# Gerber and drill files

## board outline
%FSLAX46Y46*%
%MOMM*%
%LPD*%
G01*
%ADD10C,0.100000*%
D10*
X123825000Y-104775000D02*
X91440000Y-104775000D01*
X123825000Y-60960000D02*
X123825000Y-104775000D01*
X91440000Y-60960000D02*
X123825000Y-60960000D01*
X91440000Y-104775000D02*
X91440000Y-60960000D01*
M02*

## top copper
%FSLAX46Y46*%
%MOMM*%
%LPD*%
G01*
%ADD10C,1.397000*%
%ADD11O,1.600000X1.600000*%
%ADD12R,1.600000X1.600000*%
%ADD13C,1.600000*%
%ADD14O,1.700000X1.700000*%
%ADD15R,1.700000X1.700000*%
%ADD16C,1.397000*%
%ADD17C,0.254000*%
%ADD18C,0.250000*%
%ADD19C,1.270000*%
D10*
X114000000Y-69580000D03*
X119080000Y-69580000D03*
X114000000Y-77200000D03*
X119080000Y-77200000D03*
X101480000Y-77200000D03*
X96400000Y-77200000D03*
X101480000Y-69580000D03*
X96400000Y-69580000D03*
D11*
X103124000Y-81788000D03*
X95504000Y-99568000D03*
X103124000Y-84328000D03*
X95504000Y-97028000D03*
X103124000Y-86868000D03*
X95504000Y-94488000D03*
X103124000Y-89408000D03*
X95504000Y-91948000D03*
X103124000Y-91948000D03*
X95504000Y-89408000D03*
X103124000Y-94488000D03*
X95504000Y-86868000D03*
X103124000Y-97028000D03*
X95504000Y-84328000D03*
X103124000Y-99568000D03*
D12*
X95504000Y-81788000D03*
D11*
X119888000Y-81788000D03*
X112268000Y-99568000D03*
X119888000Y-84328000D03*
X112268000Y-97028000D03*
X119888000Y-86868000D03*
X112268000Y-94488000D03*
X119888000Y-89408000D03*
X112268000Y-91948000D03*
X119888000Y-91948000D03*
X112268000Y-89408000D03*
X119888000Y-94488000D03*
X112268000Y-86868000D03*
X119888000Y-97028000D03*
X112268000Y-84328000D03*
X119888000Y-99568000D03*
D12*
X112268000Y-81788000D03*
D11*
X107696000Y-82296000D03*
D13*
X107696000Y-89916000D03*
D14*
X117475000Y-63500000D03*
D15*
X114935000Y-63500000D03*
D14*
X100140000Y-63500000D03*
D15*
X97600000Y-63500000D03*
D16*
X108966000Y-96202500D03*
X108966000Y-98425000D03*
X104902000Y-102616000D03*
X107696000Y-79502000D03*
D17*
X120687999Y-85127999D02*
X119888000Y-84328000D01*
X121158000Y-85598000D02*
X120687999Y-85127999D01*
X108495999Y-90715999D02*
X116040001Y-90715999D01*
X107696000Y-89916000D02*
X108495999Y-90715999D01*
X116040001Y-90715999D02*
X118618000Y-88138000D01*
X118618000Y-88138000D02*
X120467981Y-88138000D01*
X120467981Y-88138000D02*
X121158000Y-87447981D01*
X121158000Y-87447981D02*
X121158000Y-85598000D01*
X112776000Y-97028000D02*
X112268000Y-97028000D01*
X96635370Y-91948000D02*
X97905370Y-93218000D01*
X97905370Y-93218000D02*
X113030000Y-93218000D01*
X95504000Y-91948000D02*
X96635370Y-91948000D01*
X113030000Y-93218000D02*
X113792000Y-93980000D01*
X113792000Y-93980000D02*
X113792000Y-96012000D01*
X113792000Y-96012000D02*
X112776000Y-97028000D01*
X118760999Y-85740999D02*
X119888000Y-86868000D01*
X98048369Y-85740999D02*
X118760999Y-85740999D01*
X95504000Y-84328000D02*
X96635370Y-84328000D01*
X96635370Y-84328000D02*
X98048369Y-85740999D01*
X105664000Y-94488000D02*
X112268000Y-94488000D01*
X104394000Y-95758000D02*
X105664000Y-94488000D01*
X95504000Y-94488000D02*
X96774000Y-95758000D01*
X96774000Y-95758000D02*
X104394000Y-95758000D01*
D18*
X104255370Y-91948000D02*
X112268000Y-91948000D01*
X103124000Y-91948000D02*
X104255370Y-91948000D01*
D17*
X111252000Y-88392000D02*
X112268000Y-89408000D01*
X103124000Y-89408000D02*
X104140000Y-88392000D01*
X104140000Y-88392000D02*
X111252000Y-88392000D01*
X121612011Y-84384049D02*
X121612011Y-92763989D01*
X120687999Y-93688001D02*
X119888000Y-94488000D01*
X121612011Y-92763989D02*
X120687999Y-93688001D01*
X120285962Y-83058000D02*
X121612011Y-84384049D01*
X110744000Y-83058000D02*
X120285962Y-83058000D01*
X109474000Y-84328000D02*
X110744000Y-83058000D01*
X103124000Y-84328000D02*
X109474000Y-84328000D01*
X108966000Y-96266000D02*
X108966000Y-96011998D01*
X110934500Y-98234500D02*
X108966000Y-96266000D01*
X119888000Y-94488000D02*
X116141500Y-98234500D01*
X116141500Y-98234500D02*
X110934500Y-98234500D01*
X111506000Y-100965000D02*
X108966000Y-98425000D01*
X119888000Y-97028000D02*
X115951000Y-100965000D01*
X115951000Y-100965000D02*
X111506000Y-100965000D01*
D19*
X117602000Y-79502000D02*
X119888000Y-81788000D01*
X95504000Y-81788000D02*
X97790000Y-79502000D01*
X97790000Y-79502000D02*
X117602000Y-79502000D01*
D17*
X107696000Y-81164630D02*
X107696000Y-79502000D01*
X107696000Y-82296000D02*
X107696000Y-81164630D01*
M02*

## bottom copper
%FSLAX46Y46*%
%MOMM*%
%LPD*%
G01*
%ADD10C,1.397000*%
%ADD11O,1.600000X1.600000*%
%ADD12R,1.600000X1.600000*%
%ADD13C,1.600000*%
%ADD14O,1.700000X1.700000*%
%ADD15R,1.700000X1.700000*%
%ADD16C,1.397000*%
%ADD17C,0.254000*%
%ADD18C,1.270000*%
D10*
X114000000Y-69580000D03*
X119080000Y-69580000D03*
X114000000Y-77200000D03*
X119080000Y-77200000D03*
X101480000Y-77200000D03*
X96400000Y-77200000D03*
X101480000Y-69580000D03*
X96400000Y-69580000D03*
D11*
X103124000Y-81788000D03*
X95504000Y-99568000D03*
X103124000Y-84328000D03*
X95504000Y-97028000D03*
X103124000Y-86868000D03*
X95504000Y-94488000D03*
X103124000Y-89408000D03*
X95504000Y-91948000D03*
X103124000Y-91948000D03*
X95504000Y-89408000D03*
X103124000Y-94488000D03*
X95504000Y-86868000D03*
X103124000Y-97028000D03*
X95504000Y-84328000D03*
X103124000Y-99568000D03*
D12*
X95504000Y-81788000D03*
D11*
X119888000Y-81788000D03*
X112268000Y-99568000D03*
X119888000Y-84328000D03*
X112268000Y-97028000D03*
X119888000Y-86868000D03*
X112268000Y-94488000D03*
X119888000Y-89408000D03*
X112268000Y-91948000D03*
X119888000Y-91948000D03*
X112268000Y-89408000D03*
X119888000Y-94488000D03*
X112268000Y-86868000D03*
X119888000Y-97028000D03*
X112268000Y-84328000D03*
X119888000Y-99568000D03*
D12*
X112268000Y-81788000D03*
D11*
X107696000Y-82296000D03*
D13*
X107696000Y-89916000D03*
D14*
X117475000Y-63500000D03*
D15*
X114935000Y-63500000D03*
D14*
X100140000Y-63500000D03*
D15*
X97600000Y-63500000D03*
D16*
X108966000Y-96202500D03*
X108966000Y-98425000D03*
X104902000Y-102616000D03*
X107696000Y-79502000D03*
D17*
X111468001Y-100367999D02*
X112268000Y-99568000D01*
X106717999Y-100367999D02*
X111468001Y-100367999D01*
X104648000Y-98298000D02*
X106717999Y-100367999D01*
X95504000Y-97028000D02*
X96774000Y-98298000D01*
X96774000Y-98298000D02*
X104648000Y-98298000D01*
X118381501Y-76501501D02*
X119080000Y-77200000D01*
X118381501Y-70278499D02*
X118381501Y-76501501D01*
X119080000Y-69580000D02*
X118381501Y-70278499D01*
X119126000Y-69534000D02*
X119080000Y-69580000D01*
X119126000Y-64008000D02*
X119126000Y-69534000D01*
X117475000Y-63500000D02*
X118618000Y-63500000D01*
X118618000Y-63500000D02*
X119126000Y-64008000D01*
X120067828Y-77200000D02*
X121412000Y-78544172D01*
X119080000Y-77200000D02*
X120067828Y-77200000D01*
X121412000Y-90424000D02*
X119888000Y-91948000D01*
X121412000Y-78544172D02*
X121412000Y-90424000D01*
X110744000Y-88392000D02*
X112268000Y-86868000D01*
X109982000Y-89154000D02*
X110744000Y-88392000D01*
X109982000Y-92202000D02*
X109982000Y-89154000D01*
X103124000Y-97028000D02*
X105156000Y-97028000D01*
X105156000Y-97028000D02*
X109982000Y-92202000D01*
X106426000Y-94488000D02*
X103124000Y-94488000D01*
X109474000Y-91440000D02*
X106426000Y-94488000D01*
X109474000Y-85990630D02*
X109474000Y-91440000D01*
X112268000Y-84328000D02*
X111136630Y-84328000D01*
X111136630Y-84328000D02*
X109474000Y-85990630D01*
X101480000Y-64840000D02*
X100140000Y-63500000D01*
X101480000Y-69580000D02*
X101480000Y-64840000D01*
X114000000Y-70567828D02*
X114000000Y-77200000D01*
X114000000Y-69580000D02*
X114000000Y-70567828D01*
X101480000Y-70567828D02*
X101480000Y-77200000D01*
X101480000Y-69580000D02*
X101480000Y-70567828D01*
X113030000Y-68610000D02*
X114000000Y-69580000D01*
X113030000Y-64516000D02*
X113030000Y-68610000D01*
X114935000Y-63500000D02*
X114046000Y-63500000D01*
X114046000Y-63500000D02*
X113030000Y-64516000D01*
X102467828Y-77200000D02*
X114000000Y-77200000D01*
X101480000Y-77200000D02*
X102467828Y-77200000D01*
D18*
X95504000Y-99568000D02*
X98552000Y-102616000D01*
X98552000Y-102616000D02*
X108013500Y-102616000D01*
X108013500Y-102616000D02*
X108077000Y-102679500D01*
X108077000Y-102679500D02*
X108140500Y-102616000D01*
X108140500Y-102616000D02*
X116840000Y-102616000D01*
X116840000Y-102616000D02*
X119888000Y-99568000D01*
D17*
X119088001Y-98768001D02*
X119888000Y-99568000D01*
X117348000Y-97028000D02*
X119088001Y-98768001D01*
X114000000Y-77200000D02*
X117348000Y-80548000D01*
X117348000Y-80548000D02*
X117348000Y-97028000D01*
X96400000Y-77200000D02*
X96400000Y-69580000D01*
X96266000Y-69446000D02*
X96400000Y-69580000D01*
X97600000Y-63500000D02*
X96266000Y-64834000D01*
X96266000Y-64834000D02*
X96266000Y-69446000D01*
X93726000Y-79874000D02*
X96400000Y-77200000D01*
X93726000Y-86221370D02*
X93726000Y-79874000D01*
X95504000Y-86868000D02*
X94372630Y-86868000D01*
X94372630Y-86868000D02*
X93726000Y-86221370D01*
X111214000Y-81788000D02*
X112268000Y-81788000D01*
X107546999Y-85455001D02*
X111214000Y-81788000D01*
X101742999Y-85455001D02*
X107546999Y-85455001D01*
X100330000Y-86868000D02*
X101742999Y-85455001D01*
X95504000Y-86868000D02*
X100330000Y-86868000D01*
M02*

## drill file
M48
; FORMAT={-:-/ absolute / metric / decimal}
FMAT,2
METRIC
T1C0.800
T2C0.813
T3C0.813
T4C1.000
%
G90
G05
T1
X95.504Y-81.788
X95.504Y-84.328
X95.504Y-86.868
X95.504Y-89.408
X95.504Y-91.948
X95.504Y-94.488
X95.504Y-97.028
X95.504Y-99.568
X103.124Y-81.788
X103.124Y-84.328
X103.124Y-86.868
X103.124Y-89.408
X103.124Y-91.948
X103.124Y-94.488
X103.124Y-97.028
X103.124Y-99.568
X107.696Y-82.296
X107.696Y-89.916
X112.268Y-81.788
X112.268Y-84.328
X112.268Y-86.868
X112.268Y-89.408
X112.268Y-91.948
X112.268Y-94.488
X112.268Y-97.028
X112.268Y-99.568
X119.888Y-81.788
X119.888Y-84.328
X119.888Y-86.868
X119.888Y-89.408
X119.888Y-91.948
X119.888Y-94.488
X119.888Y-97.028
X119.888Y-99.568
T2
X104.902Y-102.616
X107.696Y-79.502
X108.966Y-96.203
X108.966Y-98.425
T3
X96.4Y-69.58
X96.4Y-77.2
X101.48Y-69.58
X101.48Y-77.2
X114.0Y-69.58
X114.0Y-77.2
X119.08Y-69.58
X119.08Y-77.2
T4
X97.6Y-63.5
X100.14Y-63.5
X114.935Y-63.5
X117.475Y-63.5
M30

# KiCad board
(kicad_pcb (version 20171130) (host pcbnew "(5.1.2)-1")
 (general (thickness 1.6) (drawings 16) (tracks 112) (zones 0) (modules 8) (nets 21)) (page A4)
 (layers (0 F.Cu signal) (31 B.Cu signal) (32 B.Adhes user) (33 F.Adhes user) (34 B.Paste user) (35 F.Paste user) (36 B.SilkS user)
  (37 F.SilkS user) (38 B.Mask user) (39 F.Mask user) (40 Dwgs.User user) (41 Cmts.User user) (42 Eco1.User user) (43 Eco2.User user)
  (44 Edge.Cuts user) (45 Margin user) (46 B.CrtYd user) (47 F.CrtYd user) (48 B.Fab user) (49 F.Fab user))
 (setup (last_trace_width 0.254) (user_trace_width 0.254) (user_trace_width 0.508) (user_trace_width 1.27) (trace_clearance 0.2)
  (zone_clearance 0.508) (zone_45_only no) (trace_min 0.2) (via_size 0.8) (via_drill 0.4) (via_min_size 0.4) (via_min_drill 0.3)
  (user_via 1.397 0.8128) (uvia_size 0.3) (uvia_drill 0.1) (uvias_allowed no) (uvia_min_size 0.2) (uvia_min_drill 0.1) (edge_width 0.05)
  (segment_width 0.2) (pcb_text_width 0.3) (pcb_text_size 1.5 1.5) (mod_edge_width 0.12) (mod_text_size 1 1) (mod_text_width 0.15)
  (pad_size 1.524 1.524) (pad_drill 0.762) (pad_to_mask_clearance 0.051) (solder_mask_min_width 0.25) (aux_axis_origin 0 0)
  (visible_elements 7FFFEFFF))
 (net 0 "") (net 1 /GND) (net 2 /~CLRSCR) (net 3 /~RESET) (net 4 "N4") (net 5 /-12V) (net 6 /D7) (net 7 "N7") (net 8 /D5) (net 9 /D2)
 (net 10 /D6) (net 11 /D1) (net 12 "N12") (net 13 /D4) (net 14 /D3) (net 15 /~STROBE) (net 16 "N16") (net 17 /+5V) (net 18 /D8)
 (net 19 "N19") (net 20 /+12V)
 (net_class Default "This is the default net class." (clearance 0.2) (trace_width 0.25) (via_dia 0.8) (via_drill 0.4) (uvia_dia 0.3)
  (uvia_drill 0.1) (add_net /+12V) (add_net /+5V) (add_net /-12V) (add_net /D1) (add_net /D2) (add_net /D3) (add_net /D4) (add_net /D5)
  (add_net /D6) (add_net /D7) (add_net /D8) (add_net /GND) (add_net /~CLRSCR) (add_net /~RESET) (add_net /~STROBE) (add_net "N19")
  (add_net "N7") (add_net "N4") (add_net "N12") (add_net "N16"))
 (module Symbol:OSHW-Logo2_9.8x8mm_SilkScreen (layer F.Cu) (at 107.2388 71.1454 90)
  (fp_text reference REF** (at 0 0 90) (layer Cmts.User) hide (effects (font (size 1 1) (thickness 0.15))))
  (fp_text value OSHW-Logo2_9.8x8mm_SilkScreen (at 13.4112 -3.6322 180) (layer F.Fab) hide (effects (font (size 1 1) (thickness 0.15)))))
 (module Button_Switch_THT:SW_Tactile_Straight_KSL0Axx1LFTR (layer F.Cu) (at 114 77.2 90)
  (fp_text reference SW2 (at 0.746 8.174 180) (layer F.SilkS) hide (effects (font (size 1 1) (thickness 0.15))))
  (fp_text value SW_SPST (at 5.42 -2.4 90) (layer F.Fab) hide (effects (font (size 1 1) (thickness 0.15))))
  (pad 1 thru_hole circle (at 7.62 0 90) (size 1.397 1.397) (drill 0.8128) (layers *.Cu *.Mask) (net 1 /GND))
  (pad 2 thru_hole circle (at 7.62 5.08 90) (size 1.397 1.397) (drill 0.8128) (layers *.Cu *.Mask) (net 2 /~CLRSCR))
  (pad 1 thru_hole circle (at 0 0 90) (size 1.397 1.397) (drill 0.8128) (layers *.Cu *.Mask) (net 1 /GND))
  (pad 2 thru_hole circle (at 0 5.08 90) (size 1.397 1.397) (drill 0.8128) (layers *.Cu *.Mask) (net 2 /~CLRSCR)))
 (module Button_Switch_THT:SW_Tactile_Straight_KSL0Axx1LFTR (layer F.Cu) (at 96.4 77.2 90)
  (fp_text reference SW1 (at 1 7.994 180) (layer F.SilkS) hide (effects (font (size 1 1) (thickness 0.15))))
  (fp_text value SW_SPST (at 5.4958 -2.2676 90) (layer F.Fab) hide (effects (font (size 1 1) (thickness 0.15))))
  (pad 2 thru_hole circle (at 0 5.08 90) (size 1.397 1.397) (drill 0.8128) (layers *.Cu *.Mask) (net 1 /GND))
  (pad 1 thru_hole circle (at 0 0 90) (size 1.397 1.397) (drill 0.8128) (layers *.Cu *.Mask) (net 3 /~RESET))
  (pad 2 thru_hole circle (at 7.62 5.08 90) (size 1.397 1.397) (drill 0.8128) (layers *.Cu *.Mask) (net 1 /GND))
  (pad 1 thru_hole circle (at 7.62 0 90) (size 1.397 1.397) (drill 0.8128) (layers *.Cu *.Mask) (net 3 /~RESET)))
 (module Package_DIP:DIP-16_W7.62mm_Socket (layer F.Cu) (at 95.504 81.788)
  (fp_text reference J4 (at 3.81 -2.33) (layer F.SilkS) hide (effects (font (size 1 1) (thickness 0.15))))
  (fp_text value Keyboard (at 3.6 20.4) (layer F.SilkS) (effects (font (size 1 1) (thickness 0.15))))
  (pad 16 thru_hole oval (at 7.62 0) (size 1.6 1.6) (drill 0.8) (layers *.Cu *.Mask) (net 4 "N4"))
  (pad 8 thru_hole oval (at 0 17.78) (size 1.6 1.6) (drill 0.8) (layers *.Cu *.Mask) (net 1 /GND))
  (pad 15 thru_hole oval (at 7.62 2.54) (size 1.6 1.6) (drill 0.8) (layers *.Cu *.Mask) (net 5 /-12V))
  (pad 7 thru_hole oval (at 0 15.24) (size 1.6 1.6) (drill 0.8) (layers *.Cu *.Mask) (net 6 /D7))
  (pad 14 thru_hole oval (at 7.62 5.08) (size 1.6 1.6) (drill 0.8) (layers *.Cu *.Mask) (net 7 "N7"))
  (pad 6 thru_hole oval (at 0 12.7) (size 1.6 1.6) (drill 0.8) (layers *.Cu *.Mask) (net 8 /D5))
  (pad 13 thru_hole oval (at 7.62 7.62) (size 1.6 1.6) (drill 0.8) (layers *.Cu *.Mask) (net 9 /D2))
  (pad 5 thru_hole oval (at 0 10.16) (size 1.6 1.6) (drill 0.8) (layers *.Cu *.Mask) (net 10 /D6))
  (pad 12 thru_hole oval (at 7.62 10.16) (size 1.6 1.6) (drill 0.8) (layers *.Cu *.Mask) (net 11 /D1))
  (pad 4 thru_hole oval (at 0 7.62) (size 1.6 1.6) (drill 0.8) (layers *.Cu *.Mask) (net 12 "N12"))
  (pad 11 thru_hole oval (at 7.62 12.7) (size 1.6 1.6) (drill 0.8) (layers *.Cu *.Mask) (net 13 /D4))
  (pad 3 thru_hole oval (at 0 5.08) (size 1.6 1.6) (drill 0.8) (layers *.Cu *.Mask) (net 3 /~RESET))
  (pad 10 thru_hole oval (at 7.62 15.24) (size 1.6 1.6) (drill 0.8) (layers *.Cu *.Mask) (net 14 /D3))
  (pad 2 thru_hole oval (at 0 2.54) (size 1.6 1.6) (drill 0.8) (layers *.Cu *.Mask) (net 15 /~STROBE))
  (pad 9 thru_hole oval (at 7.62 17.78) (size 1.6 1.6) (drill 0.8) (layers *.Cu *.Mask) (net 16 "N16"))
  (pad 1 thru_hole rect (at 0 0) (size 1.6 1.6) (drill 0.8) (layers *.Cu *.Mask) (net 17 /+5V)))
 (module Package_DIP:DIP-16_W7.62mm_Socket (layer F.Cu) (at 112.268 81.788)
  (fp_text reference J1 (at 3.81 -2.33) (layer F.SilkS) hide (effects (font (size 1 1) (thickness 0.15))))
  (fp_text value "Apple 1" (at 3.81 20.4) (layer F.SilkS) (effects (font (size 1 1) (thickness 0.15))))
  (pad 16 thru_hole oval (at 7.62 0) (size 1.6 1.6) (drill 0.8) (layers *.Cu *.Mask) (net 17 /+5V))
  (pad 8 thru_hole oval (at 0 17.78) (size 1.6 1.6) (drill 0.8) (layers *.Cu *.Mask) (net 6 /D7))
  (pad 15 thru_hole oval (at 7.62 2.54) (size 1.6 1.6) (drill 0.8) (layers *.Cu *.Mask) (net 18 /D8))
  (pad 7 thru_hole oval (at 0 15.24) (size 1.6 1.6) (drill 0.8) (layers *.Cu *.Mask) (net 10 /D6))
  (pad 14 thru_hole oval (at 7.62 5.08) (size 1.6 1.6) (drill 0.8) (layers *.Cu *.Mask) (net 15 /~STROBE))
  (pad 6 thru_hole oval (at 0 12.7) (size 1.6 1.6) (drill 0.8) (layers *.Cu *.Mask) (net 8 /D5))
  (pad 13 thru_hole oval (at 7.62 7.62) (size 1.6 1.6) (drill 0.8) (layers *.Cu *.Mask) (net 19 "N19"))
  (pad 5 thru_hole oval (at 0 10.16) (size 1.6 1.6) (drill 0.8) (layers *.Cu *.Mask) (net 11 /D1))
  (pad 12 thru_hole oval (at 7.62 10.16) (size 1.6 1.6) (drill 0.8) (layers *.Cu *.Mask) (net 2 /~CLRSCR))
  (pad 4 thru_hole oval (at 0 7.62) (size 1.6 1.6) (drill 0.8) (layers *.Cu *.Mask) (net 9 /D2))
  (pad 11 thru_hole oval (at 7.62 12.7) (size 1.6 1.6) (drill 0.8) (layers *.Cu *.Mask) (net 5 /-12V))
  (pad 3 thru_hole oval (at 0 5.08) (size 1.6 1.6) (drill 0.8) (layers *.Cu *.Mask) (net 14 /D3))
  (pad 10 thru_hole oval (at 7.62 15.24) (size 1.6 1.6) (drill 0.8) (layers *.Cu *.Mask) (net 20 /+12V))
  (pad 2 thru_hole oval (at 0 2.54) (size 1.6 1.6) (drill 0.8) (layers *.Cu *.Mask) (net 13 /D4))
  (pad 9 thru_hole oval (at 7.62 17.78) (size 1.6 1.6) (drill 0.8) (layers *.Cu *.Mask) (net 1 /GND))
  (pad 1 thru_hole rect (at 0 0) (size 1.6 1.6) (drill 0.8) (layers *.Cu *.Mask) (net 3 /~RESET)))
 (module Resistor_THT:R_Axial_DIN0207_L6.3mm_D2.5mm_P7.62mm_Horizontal (layer F.Cu) (at 107.696 89.916 90)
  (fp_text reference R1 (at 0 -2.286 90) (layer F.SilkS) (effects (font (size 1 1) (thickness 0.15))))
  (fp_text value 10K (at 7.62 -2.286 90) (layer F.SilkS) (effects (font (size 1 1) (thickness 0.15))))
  (pad 2 thru_hole oval (at 7.62 0 90) (size 1.6 1.6) (drill 0.8) (layers *.Cu *.Mask) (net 17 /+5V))
  (pad 1 thru_hole circle (at 0 0 90) (size 1.6 1.6) (drill 0.8) (layers *.Cu *.Mask) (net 18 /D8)))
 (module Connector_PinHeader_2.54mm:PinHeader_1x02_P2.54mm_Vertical (layer F.Cu) (at 114.935 63.5 90)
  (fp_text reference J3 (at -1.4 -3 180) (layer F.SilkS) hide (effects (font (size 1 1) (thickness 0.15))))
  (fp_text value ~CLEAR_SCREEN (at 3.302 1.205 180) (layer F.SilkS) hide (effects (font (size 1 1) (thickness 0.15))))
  (pad 2 thru_hole oval (at 0 2.54 90) (size 1.7 1.7) (drill 1) (layers *.Cu *.Mask) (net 2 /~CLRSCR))
  (pad 1 thru_hole rect (at 0 0 90) (size 1.7 1.7) (drill 1) (layers *.Cu *.Mask) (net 1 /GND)))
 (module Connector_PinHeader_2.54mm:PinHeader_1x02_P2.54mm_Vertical (layer F.Cu) (at 97.6 63.5 90)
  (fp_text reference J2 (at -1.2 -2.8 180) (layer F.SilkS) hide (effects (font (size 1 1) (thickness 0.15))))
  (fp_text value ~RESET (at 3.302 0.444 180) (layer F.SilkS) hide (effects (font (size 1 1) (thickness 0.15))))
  (pad 2 thru_hole oval (at 0 2.54 90) (size 1.7 1.7) (drill 1) (layers *.Cu *.Mask) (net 1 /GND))
  (pad 1 thru_hole rect (at 0 0 90) (size 1.7 1.7) (drill 1) (layers *.Cu *.Mask) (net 3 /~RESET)))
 (gr_line (start 123.825 104.775) (end 91.44 104.775) (layer Edge.Cuts) (width 0.1))
 (gr_line (start 123.825 60.96) (end 123.825 104.775) (layer Edge.Cuts) (width 0.1))
 (gr_line (start 91.44 60.96) (end 123.825 60.96) (layer Edge.Cuts) (width 0.1))
 (gr_line (start 91.44 104.775) (end 91.44 60.96) (layer Edge.Cuts) (width 0.1))
 (segment (start 111.468001 100.367999) (end 112.268 99.568) (width 0.254) (layer B.Cu) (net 6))
 (segment (start 106.717999 100.367999) (end 111.468001 100.367999) (width 0.254) (layer B.Cu) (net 6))
 (segment (start 104.648 98.298) (end 106.717999 100.367999) (width 0.254) (layer B.Cu) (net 6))
 (segment (start 95.504 97.028) (end 96.774 98.298) (width 0.254) (layer B.Cu) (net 6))
 (segment (start 96.774 98.298) (end 104.648 98.298) (width 0.254) (layer B.Cu) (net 6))
 (segment (start 120.687999 85.127999) (end 119.888 84.328) (width 0.254) (layer F.Cu) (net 18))
 (segment (start 121.158 85.598) (end 120.687999 85.127999) (width 0.254) (layer F.Cu) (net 18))
 (segment (start 108.495999 90.715999) (end 116.040001 90.715999) (width 0.254) (layer F.Cu) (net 18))
 (segment (start 107.696 89.916) (end 108.495999 90.715999) (width 0.254) (layer F.Cu) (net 18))
 (segment (start 116.040001 90.715999) (end 118.618 88.138) (width 0.254) (layer F.Cu) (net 18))
 (segment (start 118.618 88.138) (end 120.467981 88.138) (width 0.254) (layer F.Cu) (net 18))
 (segment (start 120.467981 88.138) (end 121.158 87.447981) (width 0.254) (layer F.Cu) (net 18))
 (segment (start 121.158 87.447981) (end 121.158 85.598) (width 0.254) (layer F.Cu) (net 18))
 (segment (start 112.776 97.028) (end 112.268 97.028) (width 0.254) (layer F.Cu) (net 10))
 (segment (start 96.63537 91.948) (end 97.90537 93.218) (width 0.254) (layer F.Cu) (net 10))
 (segment (start 97.90537 93.218) (end 113.03 93.218) (width 0.254) (layer F.Cu) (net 10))
 (segment (start 95.504 91.948) (end 96.63537 91.948) (width 0.254) (layer F.Cu) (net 10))
 (segment (start 113.03 93.218) (end 113.792 93.98) (width 0.254) (layer F.Cu) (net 10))
 (segment (start 113.792 93.98) (end 113.792 96.012) (width 0.254) (layer F.Cu) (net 10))
 (segment (start 113.792 96.012) (end 112.776 97.028) (width 0.254) (layer F.Cu) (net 10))
 (segment (start 118.760999 85.740999) (end 119.888 86.868) (width 0.254) (layer F.Cu) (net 15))
 (segment (start 98.048369 85.740999) (end 118.760999 85.740999) (width 0.254) (layer F.Cu) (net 15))
 (segment (start 95.504 84.328) (end 96.63537 84.328) (width 0.254) (layer F.Cu) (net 15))
 (segment (start 96.63537 84.328) (end 98.048369 85.740999) (width 0.254) (layer F.Cu) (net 15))
 (segment (start 105.664 94.488) (end 112.268 94.488) (width 0.254) (layer F.Cu) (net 8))
 (segment (start 104.394 95.758) (end 105.664 94.488) (width 0.254) (layer F.Cu) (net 8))
 (segment (start 95.504 94.488) (end 96.774 95.758) (width 0.254) (layer F.Cu) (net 8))
 (segment (start 96.774 95.758) (end 104.394 95.758) (width 0.254) (layer F.Cu) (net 8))
 (segment (start 104.25537 91.948) (end 112.268 91.948) (width 0.25) (layer F.Cu) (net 11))
 (segment (start 103.124 91.948) (end 104.25537 91.948) (width 0.25) (layer F.Cu) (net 11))
 (segment (start 118.381501 76.501501) (end 119.08 77.2) (width 0.254) (layer B.Cu) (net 2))
 (segment (start 118.381501 70.278499) (end 118.381501 76.501501) (width 0.254) (layer B.Cu) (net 2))
 (segment (start 119.08 69.58) (end 118.381501 70.278499) (width 0.254) (layer B.Cu) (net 2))
 (segment (start 119.126 69.534) (end 119.08 69.58) (width 0.254) (layer B.Cu) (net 2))
 (segment (start 119.126 64.008) (end 119.126 69.534) (width 0.254) (layer B.Cu) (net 2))
 (segment (start 117.475 63.5) (end 118.618 63.5) (width 0.254) (layer B.Cu) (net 2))
 (segment (start 118.618 63.5) (end 119.126 64.008) (width 0.254) (layer B.Cu) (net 2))
 (segment (start 120.067828 77.2) (end 121.412 78.544172) (width 0.254) (layer B.Cu) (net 2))
 (segment (start 119.08 77.2) (end 120.067828 77.2) (width 0.254) (layer B.Cu) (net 2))
 (segment (start 121.412 90.424) (end 119.888 91.948) (width 0.254) (layer B.Cu) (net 2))
 (segment (start 121.412 78.544172) (end 121.412 90.424) (width 0.254) (layer B.Cu) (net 2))
 (segment (start 111.252 88.392) (end 112.268 89.408) (width 0.254) (layer F.Cu) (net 9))
 (segment (start 103.124 89.408) (end 104.14 88.392) (width 0.254) (layer F.Cu) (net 9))
 (segment (start 104.14 88.392) (end 111.252 88.392) (width 0.254) (layer F.Cu) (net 9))
 (segment (start 121.612011 84.384049) (end 121.612011 92.763989) (width 0.254) (layer F.Cu) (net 5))
 (segment (start 120.687999 93.688001) (end 119.888 94.488) (width 0.254) (layer F.Cu) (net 5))
 (segment (start 121.612011 92.763989) (end 120.687999 93.688001) (width 0.254) (layer F.Cu) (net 5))
 (segment (start 120.285962 83.058) (end 121.612011 84.384049) (width 0.254) (layer F.Cu) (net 5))
 (segment (start 110.744 83.058) (end 120.285962 83.058) (width 0.254) (layer F.Cu) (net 5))
 (segment (start 109.474 84.328) (end 110.744 83.058) (width 0.254) (layer F.Cu) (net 5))
 (segment (start 103.124 84.328) (end 109.474 84.328) (width 0.254) (layer F.Cu) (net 5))
 (via (at 108.966 96.2025) (size 1.397) (drill 0.8128) (layers F.Cu B.Cu) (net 5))
 (segment (start 108.966 96.266) (end 108.966 96.011998) (width 0.254) (layer F.Cu) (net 5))
 (segment (start 110.9345 98.2345) (end 108.966 96.266) (width 0.254) (layer F.Cu) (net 5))
 (segment (start 119.888 94.488) (end 116.1415 98.2345) (width 0.254) (layer F.Cu) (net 5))
 (segment (start 116.1415 98.2345) (end 110.9345 98.2345) (width 0.254) (layer F.Cu) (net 5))
 (segment (start 110.744 88.392) (end 112.268 86.868) (width 0.254) (layer B.Cu) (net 14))
 (segment (start 109.982 89.154) (end 110.744 88.392) (width 0.254) (layer B.Cu) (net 14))
 (segment (start 109.982 92.202) (end 109.982 89.154) (width 0.254) (layer B.Cu) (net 14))
 (segment (start 103.124 97.028) (end 105.156 97.028) (width 0.254) (layer B.Cu) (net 14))
 (segment (start 105.156 97.028) (end 109.982 92.202) (width 0.254) (layer B.Cu) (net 14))
 (via (at 108.966 98.425) (size 1.397) (drill 0.8128) (layers F.Cu B.Cu) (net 20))
 (segment (start 111.506 100.965) (end 108.966 98.425) (width 0.254) (layer F.Cu) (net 20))
 (segment (start 119.888 97.028) (end 115.951 100.965) (width 0.254) (layer F.Cu) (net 20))
 (segment (start 115.951 100.965) (end 111.506 100.965) (width 0.254) (layer F.Cu) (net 20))
 (segment (start 106.426 94.488) (end 103.124 94.488) (width 0.254) (layer B.Cu) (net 13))
 (segment (start 109.474 91.44) (end 106.426 94.488) (width 0.254) (layer B.Cu) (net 13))
 (segment (start 109.474 85.99063) (end 109.474 91.44) (width 0.254) (layer B.Cu) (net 13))
 (segment (start 112.268 84.328) (end 111.13663 84.328) (width 0.254) (layer B.Cu) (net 13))
 (segment (start 111.13663 84.328) (end 109.474 85.99063) (width 0.254) (layer B.Cu) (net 13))
 (segment (start 101.48 64.84) (end 100.14 63.5) (width 0.254) (layer B.Cu) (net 1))
 (segment (start 101.48 69.58) (end 101.48 64.84) (width 0.254) (layer B.Cu) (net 1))
 (segment (start 114 70.567828) (end 114 77.2) (width 0.254) (layer B.Cu) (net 1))
 (segment (start 114 69.58) (end 114 70.567828) (width 0.254) (layer B.Cu) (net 1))
 (segment (start 101.48 70.567828) (end 101.48 77.2) (width 0.254) (layer B.Cu) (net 1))
 (segment (start 101.48 69.58) (end 101.48 70.567828) (width 0.254) (layer B.Cu) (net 1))
 (segment (start 113.03 68.61) (end 114 69.58) (width 0.254) (layer B.Cu) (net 1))
 (segment (start 113.03 64.516) (end 113.03 68.61) (width 0.254) (layer B.Cu) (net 1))
 (segment (start 114.935 63.5) (end 114.046 63.5) (width 0.254) (layer B.Cu) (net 1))
 (segment (start 114.046 63.5) (end 113.03 64.516) (width 0.254) (layer B.Cu) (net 1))
 (segment (start 102.467828 77.2) (end 114 77.2) (width 0.254) (layer B.Cu) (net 1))
 (segment (start 101.48 77.2) (end 102.467828 77.2) (width 0.254) (layer B.Cu) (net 1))
 (segment (start 95.504 99.568) (end 98.552 102.616) (width 1.27) (layer B.Cu) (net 1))
 (segment (start 98.552 102.616) (end 108.0135 102.616) (width 1.27) (layer B.Cu) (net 1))
 (segment (start 108.0135 102.616) (end 108.077 102.6795) (width 1.27) (layer B.Cu) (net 1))
 (segment (start 108.077 102.6795) (end 108.1405 102.616) (width 1.27) (layer B.Cu) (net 1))
 (segment (start 108.1405 102.616) (end 116.84 102.616) (width 1.27) (layer B.Cu) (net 1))
 (segment (start 116.84 102.616) (end 119.888 99.568) (width 1.27) (layer B.Cu) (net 1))
 (via (at 104.902 102.616) (size 1.397) (drill 0.8128) (layers F.Cu B.Cu) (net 1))
 (segment (start 119.088001 98.768001) (end 119.888 99.568) (width 0.254) (layer B.Cu) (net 1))
 (segment (start 117.348 97.028) (end 119.088001 98.768001) (width 0.254) (layer B.Cu) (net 1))
 (segment (start 114 77.2) (end 117.348 80.548) (width 0.254) (layer B.Cu) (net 1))
 (segment (start 117.348 80.548) (end 117.348 97.028) (width 0.254) (layer B.Cu) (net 1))
 (segment (start 96.4 77.2) (end 96.4 69.58) (width 0.254) (layer B.Cu) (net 3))
 (segment (start 96.266 69.446) (end 96.4 69.58) (width 0.254) (layer B.Cu) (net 3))
 (segment (start 97.6 63.5) (end 96.266 64.834) (width 0.254) (layer B.Cu) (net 3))
 (segment (start 96.266 64.834) (end 96.266 69.446) (width 0.254) (layer B.Cu) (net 3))
 (segment (start 93.726 79.874) (end 96.4 77.2) (width 0.254) (layer B.Cu) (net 3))
 (segment (start 93.726 86.22137) (end 93.726 79.874) (width 0.254) (layer B.Cu) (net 3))
 (segment (start 95.504 86.868) (end 94.37263 86.868) (width 0.254) (layer B.Cu) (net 3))
 (segment (start 94.37263 86.868) (end 93.726 86.22137) (width 0.254) (layer B.Cu) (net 3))
 (segment (start 111.214 81.788) (end 112.268 81.788) (width 0.254) (layer B.Cu) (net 3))
 (segment (start 107.546999 85.455001) (end 111.214 81.788) (width 0.254) (layer B.Cu) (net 3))
 (segment (start 101.742999 85.455001) (end 107.546999 85.455001) (width 0.254) (layer B.Cu) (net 3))
 (segment (start 100.33 86.868) (end 101.742999 85.455001) (width 0.254) (layer B.Cu) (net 3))
 (segment (start 95.504 86.868) (end 100.33 86.868) (width 0.254) (layer B.Cu) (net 3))
 (via (at 107.696 79.502) (size 1.397) (drill 0.8128) (layers F.Cu B.Cu) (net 17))
 (segment (start 117.602 79.502) (end 119.888 81.788) (width 1.27) (layer F.Cu) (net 17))
 (segment (start 95.504 81.788) (end 97.79 79.502) (width 1.27) (layer F.Cu) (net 17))
 (segment (start 97.79 79.502) (end 117.602 79.502) (width 1.27) (layer F.Cu) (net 17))
 (segment (start 107.696 81.16463) (end 107.696 79.502) (width 0.254) (layer F.Cu) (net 17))
 (segment (start 107.696 82.296) (end 107.696 81.16463) (width 0.254) (layer F.Cu) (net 17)))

